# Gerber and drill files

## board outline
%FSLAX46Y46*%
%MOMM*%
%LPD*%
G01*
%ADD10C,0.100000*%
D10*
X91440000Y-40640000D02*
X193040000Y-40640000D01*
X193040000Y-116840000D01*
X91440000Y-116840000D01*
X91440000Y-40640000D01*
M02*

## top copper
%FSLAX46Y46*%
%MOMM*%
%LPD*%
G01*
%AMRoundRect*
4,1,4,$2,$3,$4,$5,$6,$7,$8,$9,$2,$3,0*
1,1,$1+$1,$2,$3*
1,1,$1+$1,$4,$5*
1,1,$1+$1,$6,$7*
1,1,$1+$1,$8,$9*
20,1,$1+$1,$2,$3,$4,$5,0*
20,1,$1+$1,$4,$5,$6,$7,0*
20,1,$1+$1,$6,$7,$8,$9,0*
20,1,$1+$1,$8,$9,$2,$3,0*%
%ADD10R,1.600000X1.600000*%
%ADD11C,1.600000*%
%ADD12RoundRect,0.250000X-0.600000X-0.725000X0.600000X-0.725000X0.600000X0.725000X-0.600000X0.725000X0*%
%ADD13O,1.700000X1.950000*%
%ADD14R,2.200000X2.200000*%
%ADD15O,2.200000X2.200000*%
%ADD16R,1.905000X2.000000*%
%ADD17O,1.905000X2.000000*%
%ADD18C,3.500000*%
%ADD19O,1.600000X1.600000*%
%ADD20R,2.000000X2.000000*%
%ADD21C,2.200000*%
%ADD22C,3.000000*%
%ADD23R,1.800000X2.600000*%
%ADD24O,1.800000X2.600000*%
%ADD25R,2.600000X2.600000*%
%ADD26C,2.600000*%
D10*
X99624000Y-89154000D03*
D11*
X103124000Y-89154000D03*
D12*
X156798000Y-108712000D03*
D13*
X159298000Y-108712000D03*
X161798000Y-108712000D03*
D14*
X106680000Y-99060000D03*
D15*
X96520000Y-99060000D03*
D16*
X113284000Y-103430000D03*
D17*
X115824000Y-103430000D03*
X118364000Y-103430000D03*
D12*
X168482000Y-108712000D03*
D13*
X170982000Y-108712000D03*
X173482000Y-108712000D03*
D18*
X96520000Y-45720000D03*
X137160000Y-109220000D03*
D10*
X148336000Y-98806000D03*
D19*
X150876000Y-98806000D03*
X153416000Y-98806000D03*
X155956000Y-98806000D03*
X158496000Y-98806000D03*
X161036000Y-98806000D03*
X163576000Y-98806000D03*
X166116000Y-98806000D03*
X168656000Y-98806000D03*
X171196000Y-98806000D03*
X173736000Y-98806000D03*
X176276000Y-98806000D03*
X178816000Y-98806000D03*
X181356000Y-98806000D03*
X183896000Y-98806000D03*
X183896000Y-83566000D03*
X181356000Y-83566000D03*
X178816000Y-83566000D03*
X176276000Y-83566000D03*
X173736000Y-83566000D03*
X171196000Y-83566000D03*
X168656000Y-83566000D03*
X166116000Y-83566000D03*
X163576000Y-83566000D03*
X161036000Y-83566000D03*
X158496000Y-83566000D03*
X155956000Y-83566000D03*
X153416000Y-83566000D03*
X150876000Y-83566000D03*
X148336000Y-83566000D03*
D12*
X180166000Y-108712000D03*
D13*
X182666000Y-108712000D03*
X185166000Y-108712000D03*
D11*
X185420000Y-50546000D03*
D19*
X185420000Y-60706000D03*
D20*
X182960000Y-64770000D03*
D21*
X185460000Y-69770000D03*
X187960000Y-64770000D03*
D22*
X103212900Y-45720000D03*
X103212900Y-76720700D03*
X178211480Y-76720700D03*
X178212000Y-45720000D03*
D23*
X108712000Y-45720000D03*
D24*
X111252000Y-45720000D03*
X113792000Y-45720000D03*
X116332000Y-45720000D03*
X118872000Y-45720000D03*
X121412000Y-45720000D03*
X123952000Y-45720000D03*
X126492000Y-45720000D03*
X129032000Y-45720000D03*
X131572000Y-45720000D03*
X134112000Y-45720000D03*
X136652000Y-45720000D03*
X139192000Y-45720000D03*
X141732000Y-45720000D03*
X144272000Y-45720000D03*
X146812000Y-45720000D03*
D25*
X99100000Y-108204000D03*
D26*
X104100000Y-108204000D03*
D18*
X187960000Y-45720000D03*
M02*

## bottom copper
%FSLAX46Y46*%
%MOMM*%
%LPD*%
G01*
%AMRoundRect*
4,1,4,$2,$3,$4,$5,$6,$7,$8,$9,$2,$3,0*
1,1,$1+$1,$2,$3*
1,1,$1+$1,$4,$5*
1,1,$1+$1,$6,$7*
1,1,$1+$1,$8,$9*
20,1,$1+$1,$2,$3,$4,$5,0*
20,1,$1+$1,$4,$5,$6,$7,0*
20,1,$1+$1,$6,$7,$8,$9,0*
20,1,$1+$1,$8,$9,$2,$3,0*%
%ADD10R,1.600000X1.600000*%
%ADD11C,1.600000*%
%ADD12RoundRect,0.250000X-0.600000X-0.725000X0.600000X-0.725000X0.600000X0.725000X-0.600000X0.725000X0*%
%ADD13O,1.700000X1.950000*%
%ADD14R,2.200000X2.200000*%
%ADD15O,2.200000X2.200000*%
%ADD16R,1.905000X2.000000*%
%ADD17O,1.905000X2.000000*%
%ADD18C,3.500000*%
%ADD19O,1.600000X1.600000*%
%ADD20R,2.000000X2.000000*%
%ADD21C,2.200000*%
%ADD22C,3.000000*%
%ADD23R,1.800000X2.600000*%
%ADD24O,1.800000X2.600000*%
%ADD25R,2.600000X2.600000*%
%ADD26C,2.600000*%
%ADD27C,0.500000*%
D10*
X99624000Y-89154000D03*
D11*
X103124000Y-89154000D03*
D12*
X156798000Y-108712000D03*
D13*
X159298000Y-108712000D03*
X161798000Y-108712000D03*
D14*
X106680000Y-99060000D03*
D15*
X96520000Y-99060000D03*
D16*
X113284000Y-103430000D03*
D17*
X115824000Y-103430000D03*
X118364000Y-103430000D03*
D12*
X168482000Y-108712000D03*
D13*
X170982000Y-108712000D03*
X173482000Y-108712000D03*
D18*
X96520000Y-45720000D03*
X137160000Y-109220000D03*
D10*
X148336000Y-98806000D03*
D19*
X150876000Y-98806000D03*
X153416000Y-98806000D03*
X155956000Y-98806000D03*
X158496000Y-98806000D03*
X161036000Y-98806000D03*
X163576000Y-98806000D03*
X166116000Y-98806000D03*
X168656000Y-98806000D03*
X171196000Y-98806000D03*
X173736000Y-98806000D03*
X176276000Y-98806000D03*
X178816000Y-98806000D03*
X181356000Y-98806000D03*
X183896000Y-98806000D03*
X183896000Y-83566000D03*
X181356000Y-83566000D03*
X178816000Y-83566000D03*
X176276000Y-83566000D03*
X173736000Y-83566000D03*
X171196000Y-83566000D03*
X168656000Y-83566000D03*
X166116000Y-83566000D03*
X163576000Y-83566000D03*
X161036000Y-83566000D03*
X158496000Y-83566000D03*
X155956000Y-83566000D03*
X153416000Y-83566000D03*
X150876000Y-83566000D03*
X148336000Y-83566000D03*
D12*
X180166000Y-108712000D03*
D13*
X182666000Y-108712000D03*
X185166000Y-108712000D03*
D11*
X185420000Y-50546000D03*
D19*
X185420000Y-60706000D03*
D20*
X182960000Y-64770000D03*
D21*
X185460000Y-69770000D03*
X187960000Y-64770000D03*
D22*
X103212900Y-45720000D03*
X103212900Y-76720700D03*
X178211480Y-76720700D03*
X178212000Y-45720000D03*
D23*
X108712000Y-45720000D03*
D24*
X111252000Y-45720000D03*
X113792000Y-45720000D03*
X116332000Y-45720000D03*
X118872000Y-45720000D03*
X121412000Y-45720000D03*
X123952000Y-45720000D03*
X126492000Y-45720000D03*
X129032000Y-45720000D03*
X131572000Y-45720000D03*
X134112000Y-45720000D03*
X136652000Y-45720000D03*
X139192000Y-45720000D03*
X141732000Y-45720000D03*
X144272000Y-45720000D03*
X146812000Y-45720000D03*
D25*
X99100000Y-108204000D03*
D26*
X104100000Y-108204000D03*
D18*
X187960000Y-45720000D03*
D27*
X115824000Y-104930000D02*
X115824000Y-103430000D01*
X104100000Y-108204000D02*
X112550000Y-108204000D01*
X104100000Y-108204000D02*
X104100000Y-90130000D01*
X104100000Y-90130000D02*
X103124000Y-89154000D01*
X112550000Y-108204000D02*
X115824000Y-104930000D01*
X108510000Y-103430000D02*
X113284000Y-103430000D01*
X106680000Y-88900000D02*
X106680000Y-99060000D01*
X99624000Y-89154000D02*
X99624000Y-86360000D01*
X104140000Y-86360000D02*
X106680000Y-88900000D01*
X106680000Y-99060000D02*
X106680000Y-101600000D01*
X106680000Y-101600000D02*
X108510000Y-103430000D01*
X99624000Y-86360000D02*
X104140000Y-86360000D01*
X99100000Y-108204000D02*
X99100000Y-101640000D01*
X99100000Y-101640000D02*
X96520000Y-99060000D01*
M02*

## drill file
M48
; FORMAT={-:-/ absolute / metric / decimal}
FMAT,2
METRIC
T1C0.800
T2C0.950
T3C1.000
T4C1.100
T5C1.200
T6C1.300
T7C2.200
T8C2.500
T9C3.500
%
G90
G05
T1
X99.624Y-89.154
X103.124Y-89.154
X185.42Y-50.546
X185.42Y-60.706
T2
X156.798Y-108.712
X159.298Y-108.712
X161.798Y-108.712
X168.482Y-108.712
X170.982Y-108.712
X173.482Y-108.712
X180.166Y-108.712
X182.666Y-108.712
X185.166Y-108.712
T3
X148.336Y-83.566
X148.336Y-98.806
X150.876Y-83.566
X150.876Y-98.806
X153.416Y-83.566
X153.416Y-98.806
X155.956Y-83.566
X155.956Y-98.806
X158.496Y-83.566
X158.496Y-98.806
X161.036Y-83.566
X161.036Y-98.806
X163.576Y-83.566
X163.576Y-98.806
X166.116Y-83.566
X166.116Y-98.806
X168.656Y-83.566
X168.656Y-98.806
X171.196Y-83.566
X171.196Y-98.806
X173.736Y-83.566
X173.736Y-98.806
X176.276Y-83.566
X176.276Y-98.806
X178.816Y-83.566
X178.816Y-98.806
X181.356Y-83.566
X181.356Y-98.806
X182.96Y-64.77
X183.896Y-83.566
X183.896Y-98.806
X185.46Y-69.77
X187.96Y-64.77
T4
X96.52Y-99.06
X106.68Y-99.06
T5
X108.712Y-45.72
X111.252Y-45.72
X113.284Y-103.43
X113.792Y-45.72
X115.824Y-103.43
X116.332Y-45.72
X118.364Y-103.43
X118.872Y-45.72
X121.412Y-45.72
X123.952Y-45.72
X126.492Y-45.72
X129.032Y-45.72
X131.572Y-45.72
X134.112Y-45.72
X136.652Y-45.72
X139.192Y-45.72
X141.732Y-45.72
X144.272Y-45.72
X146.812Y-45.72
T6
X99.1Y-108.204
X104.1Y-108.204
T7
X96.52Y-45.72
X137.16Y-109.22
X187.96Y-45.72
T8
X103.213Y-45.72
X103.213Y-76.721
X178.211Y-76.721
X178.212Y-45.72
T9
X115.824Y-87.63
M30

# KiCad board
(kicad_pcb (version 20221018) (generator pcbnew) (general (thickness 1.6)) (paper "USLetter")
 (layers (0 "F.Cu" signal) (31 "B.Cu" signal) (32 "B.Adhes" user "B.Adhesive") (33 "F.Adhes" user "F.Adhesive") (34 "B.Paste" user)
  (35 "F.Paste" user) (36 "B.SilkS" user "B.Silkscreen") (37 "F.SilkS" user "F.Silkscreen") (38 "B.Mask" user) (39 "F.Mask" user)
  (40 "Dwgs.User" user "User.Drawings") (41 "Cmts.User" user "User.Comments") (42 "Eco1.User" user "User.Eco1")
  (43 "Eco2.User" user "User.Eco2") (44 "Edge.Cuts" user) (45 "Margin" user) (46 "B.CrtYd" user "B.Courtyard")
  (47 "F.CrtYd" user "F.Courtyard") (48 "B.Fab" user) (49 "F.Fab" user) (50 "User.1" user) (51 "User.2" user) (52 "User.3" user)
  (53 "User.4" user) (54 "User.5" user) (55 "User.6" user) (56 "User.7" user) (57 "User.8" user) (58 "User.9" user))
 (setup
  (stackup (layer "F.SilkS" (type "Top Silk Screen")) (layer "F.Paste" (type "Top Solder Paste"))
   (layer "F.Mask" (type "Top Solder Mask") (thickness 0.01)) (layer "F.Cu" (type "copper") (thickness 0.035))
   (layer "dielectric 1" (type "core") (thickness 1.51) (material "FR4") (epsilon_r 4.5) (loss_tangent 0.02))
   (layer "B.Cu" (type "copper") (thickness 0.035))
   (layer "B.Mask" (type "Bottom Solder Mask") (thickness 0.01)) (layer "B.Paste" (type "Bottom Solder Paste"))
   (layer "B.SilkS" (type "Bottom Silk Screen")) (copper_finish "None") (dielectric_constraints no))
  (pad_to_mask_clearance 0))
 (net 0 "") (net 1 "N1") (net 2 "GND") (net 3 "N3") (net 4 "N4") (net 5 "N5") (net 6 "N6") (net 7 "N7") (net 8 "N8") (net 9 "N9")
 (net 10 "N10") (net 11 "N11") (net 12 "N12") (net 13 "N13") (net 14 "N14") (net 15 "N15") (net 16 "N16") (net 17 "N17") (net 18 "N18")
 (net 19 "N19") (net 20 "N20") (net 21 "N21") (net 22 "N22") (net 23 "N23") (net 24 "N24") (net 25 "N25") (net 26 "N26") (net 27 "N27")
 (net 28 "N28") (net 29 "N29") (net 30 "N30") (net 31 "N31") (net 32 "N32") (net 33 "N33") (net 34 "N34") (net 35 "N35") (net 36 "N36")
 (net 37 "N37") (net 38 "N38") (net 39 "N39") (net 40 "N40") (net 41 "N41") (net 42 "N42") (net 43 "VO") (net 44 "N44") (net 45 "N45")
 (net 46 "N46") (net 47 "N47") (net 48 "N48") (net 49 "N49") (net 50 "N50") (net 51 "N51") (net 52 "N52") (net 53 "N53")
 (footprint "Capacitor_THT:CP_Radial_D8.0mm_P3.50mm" (layer "F.Cu") (at 99.624 89.154)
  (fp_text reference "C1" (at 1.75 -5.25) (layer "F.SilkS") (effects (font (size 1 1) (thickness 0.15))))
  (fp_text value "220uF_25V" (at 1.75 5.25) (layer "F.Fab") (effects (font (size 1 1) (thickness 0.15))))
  (pad "1" thru_hole rect (at 0 0) (size 1.6 1.6) (drill 0.8) (layers "*.Cu" "*.Mask") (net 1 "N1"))
  (pad "2" thru_hole circle (at 3.5 0) (size 1.6 1.6) (drill 0.8) (layers "*.Cu" "*.Mask") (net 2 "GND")))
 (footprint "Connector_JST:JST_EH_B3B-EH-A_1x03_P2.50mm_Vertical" (layer "F.Cu") (at 156.798 108.712)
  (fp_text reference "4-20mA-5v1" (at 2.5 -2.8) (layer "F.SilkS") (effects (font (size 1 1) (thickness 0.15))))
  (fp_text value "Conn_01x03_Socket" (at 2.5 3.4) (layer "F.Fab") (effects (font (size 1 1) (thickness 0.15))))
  (pad "1" thru_hole roundrect (at 0 0) (size 1.7 1.95) (drill 0.95) (layers "*.Cu" "*.Mask") (roundrect_rratio 0.147059) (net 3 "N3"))
  (pad "2" thru_hole oval (at 2.5 0) (size 1.7 1.95) (drill 0.95) (layers "*.Cu" "*.Mask") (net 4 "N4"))
  (pad "3" thru_hole oval (at 5 0) (size 1.7 1.95) (drill 0.95) (layers "*.Cu" "*.Mask") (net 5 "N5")))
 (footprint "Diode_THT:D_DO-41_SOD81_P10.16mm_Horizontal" (layer "F.Cu") (at 106.68 99.06 180)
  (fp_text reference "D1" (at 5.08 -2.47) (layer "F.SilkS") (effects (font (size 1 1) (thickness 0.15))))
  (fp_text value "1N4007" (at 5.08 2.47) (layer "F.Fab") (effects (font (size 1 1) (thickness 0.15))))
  (pad "1" thru_hole rect (at 0 0 180) (size 2.2 2.2) (drill 1.1) (layers "*.Cu" "*.Mask") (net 1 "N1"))
  (pad "2" thru_hole oval (at 10.16 0 180) (size 2.2 2.2) (drill 1.1) (layers "*.Cu" "*.Mask") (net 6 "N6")))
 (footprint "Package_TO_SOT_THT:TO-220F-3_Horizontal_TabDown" (layer "F.Cu") (at 113.284 103.43)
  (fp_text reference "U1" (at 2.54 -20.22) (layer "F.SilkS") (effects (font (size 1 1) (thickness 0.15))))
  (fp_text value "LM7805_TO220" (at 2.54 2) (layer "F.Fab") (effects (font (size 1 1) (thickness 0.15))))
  (pad "" np_thru_hole oval (at 2.54 -15.8) (size 3.5 3.5) (drill 3.5) (layers "*.Cu" "*.Mask"))
  (pad "1" thru_hole rect (at 0 0) (size 1.905 2) (drill 1.2) (layers "*.Cu" "*.Mask") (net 1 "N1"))
  (pad "2" thru_hole oval (at 2.54 0) (size 1.905 2) (drill 1.2) (layers "*.Cu" "*.Mask") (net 2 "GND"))
  (pad "3" thru_hole oval (at 5.08 0) (size 1.905 2) (drill 1.2) (layers "*.Cu" "*.Mask") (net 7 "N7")))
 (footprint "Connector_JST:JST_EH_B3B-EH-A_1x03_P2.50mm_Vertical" (layer "F.Cu") (at 168.482 108.712)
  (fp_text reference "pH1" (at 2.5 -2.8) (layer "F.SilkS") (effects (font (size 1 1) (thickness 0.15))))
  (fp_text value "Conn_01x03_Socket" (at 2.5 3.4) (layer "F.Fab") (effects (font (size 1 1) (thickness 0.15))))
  (pad "1" thru_hole roundrect (at 0 0) (size 1.7 1.95) (drill 0.95) (layers "*.Cu" "*.Mask") (roundrect_rratio 0.147059) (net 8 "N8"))
  (pad "2" thru_hole oval (at 2.5 0) (size 1.7 1.95) (drill 0.95) (layers "*.Cu" "*.Mask") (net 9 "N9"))
  (pad "3" thru_hole oval (at 5 0) (size 1.7 1.95) (drill 0.95) (layers "*.Cu" "*.Mask") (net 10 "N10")))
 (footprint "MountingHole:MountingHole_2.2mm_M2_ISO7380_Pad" (layer "F.Cu") (at 96.52 45.72)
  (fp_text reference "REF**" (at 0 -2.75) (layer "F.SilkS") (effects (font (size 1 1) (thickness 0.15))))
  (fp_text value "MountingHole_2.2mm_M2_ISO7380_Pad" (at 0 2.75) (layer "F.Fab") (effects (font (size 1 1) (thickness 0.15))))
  (pad "1" thru_hole circle (at 0 0) (size 3.5 3.5) (drill 2.2) (layers "*.Cu" "*.Mask")))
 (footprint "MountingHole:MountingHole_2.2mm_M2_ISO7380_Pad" (layer "F.Cu") (at 137.16 109.22)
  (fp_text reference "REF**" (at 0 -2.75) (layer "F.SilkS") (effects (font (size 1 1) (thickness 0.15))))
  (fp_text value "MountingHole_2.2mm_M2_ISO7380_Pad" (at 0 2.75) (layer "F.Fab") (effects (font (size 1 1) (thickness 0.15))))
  (pad "1" thru_hole circle (at 0 0) (size 3.5 3.5) (drill 2.2) (layers "*.Cu" "*.Mask")))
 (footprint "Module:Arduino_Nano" (layer "F.Cu") (at 148.336 98.806 90)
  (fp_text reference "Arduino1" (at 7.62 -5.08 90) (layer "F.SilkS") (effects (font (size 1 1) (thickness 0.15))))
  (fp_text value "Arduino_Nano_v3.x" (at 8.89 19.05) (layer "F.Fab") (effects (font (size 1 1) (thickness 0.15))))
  (pad "1" thru_hole rect (at 0 0 90) (size 1.6 1.6) (drill 1) (layers "*.Cu" "*.Mask") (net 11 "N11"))
  (pad "2" thru_hole oval (at 0 2.54 90) (size 1.6 1.6) (drill 1) (layers "*.Cu" "*.Mask") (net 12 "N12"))
  (pad "3" thru_hole oval (at 0 5.08 90) (size 1.6 1.6) (drill 1) (layers "*.Cu" "*.Mask") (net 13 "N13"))
  (pad "4" thru_hole oval (at 0 7.62 90) (size 1.6 1.6) (drill 1) (layers "*.Cu" "*.Mask") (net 2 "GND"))
  (pad "5" thru_hole oval (at 0 10.16 90) (size 1.6 1.6) (drill 1) (layers "*.Cu" "*.Mask") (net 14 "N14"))
  (pad "6" thru_hole oval (at 0 12.7 90) (size 1.6 1.6) (drill 1) (layers "*.Cu" "*.Mask") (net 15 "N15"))
  (pad "7" thru_hole oval (at 0 15.24 90) (size 1.6 1.6) (drill 1) (layers "*.Cu" "*.Mask") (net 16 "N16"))
  (pad "8" thru_hole oval (at 0 17.78 90) (size 1.6 1.6) (drill 1) (layers "*.Cu" "*.Mask") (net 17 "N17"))
  (pad "9" thru_hole oval (at 0 20.32 90) (size 1.6 1.6) (drill 1) (layers "*.Cu" "*.Mask") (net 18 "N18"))
  (pad "10" thru_hole oval (at 0 22.86 90) (size 1.6 1.6) (drill 1) (layers "*.Cu" "*.Mask") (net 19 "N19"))
  (pad "11" thru_hole oval (at 0 25.4 90) (size 1.6 1.6) (drill 1) (layers "*.Cu" "*.Mask") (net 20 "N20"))
  (pad "12" thru_hole oval (at 0 27.94 90) (size 1.6 1.6) (drill 1) (layers "*.Cu" "*.Mask") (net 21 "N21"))
  (pad "13" thru_hole oval (at 0 30.48 90) (size 1.6 1.6) (drill 1) (layers "*.Cu" "*.Mask") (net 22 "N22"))
  (pad "14" thru_hole oval (at 0 33.02 90) (size 1.6 1.6) (drill 1) (layers "*.Cu" "*.Mask") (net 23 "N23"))
  (pad "15" thru_hole oval (at 0 35.56 90) (size 1.6 1.6) (drill 1) (layers "*.Cu" "*.Mask") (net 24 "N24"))
  (pad "16" thru_hole oval (at 15.24 35.56 90) (size 1.6 1.6) (drill 1) (layers "*.Cu" "*.Mask") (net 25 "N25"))
  (pad "17" thru_hole oval (at 15.24 33.02 90) (size 1.6 1.6) (drill 1) (layers "*.Cu" "*.Mask") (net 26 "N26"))
  (pad "18" thru_hole oval (at 15.24 30.48 90) (size 1.6 1.6) (drill 1) (layers "*.Cu" "*.Mask") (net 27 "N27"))
  (pad "19" thru_hole oval (at 15.24 27.94 90) (size 1.6 1.6) (drill 1) (layers "*.Cu" "*.Mask") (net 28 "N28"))
  (pad "20" thru_hole oval (at 15.24 25.4 90) (size 1.6 1.6) (drill 1) (layers "*.Cu" "*.Mask") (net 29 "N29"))
  (pad "21" thru_hole oval (at 15.24 22.86 90) (size 1.6 1.6) (drill 1) (layers "*.Cu" "*.Mask") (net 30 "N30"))
  (pad "22" thru_hole oval (at 15.24 20.32 90) (size 1.6 1.6) (drill 1) (layers "*.Cu" "*.Mask") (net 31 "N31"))
  (pad "23" thru_hole oval (at 15.24 17.78 90) (size 1.6 1.6) (drill 1) (layers "*.Cu" "*.Mask") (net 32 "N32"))
  (pad "24" thru_hole oval (at 15.24 15.24 90) (size 1.6 1.6) (drill 1) (layers "*.Cu" "*.Mask") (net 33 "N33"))
  (pad "25" thru_hole oval (at 15.24 12.7 90) (size 1.6 1.6) (drill 1) (layers "*.Cu" "*.Mask") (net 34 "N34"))
  (pad "26" thru_hole oval (at 15.24 10.16 90) (size 1.6 1.6) (drill 1) (layers "*.Cu" "*.Mask") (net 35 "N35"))
  (pad "27" thru_hole oval (at 15.24 7.62 90) (size 1.6 1.6) (drill 1) (layers "*.Cu" "*.Mask") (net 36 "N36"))
  (pad "28" thru_hole oval (at 15.24 5.08 90) (size 1.6 1.6) (drill 1) (layers "*.Cu" "*.Mask") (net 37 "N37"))
  (pad "29" thru_hole oval (at 15.24 2.54 90) (size 1.6 1.6) (drill 1) (layers "*.Cu" "*.Mask") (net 2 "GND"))
  (pad "30" thru_hole oval (at 15.24 0 90) (size 1.6 1.6) (drill 1) (layers "*.Cu" "*.Mask") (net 7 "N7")))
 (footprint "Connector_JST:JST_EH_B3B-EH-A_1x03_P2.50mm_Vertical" (layer "F.Cu") (at 180.166 108.712)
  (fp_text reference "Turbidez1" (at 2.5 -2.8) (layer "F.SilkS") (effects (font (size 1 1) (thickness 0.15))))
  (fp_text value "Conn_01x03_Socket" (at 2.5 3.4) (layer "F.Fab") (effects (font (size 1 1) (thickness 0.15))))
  (pad "1" thru_hole roundrect (at 0 0) (size 1.7 1.95) (drill 0.95) (layers "*.Cu" "*.Mask") (roundrect_rratio 0.147059) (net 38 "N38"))
  (pad "2" thru_hole oval (at 2.5 0) (size 1.7 1.95) (drill 0.95) (layers "*.Cu" "*.Mask") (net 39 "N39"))
  (pad "3" thru_hole oval (at 5 0) (size 1.7 1.95) (drill 0.95) (layers "*.Cu" "*.Mask") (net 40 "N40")))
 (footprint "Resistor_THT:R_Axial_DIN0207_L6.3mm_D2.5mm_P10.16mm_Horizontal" (layer "F.Cu") (at 185.42 50.546 -90)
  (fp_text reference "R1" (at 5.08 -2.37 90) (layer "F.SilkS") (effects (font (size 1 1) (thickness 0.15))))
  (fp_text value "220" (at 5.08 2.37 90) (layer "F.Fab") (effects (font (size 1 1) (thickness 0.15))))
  (pad "1" thru_hole circle (at 0 0 270) (size 1.6 1.6) (drill 0.8) (layers "*.Cu" "*.Mask") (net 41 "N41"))
  (pad "2" thru_hole oval (at 10.16 0 270) (size 1.6 1.6) (drill 0.8) (layers "*.Cu" "*.Mask") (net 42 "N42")))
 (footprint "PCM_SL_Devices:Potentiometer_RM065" (layer "F.Cu") (at 185.49 66.8)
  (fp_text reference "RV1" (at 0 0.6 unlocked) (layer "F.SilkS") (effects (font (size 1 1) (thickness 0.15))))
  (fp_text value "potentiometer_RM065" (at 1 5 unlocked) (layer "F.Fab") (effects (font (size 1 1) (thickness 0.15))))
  (pad "1" thru_hole rect (at -2.53 -2.03) (size 2 2) (drill 1) (layers "*.Cu" "*.Mask") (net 36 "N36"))
  (pad "2" thru_hole circle (at -0.03 2.97) (size 2.2 2.2) (drill 1) (layers "*.Cu" "*.Mask") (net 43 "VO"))
  (pad "3" thru_hole circle (at 2.47 -2.03) (size 2.2 2.2) (drill 1) (layers "*.Cu" "*.Mask") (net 2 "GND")))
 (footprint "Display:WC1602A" (layer "F.Cu") (at 108.712 45.72)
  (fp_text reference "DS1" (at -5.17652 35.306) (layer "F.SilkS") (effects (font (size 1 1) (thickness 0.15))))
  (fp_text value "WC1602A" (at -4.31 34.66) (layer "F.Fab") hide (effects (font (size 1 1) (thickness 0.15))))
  (pad "" thru_hole circle (at -5.4991 0) (size 3 3) (drill 2.5) (layers "*.Cu" "*.Mask"))
  (pad "" thru_hole circle (at -5.4991 31.0007) (size 3 3) (drill 2.5) (layers "*.Cu" "*.Mask"))
  (pad "" thru_hole circle (at 69.49948 31.0007) (size 3 3) (drill 2.5) (layers "*.Cu" "*.Mask"))
  (pad "" thru_hole circle (at 69.5 0) (size 3 3) (drill 2.5) (layers "*.Cu" "*.Mask"))
  (pad "1" thru_hole rect (at 0 0) (size 1.8 2.6) (drill 1.2) (layers "*.Cu" "*.Mask") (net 2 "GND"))
  (pad "2" thru_hole oval (at 2.54 0) (size 1.8 2.6) (drill 1.2) (layers "*.Cu" "*.Mask") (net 36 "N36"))
  (pad "3" thru_hole oval (at 5.08 0) (size 1.8 2.6) (drill 1.2) (layers "*.Cu" "*.Mask") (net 43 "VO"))
  (pad "4" thru_hole oval (at 7.62 0) (size 1.8 2.6) (drill 1.2) (layers "*.Cu" "*.Mask") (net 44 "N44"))
  (pad "5" thru_hole oval (at 10.16 0) (size 1.8 2.6) (drill 1.2) (layers "*.Cu" "*.Mask") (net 15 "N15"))
  (pad "6" thru_hole oval (at 12.7 0) (size 1.8 2.6) (drill 1.2) (layers "*.Cu" "*.Mask") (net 14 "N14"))
  (pad "7" thru_hole oval (at 15.24 0) (size 1.8 2.6) (drill 1.2) (layers "*.Cu" "*.Mask") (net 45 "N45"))
  (pad "8" thru_hole oval (at 17.78 0) (size 1.8 2.6) (drill 1.2) (layers "*.Cu" "*.Mask") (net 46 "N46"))
  (pad "9" thru_hole oval (at 20.32 0) (size 1.8 2.6) (drill 1.2) (layers "*.Cu" "*.Mask") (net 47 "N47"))
  (pad "10" thru_hole oval (at 22.86 0) (size 1.8 2.6) (drill 1.2) (layers "*.Cu" "*.Mask") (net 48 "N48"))
  (pad "11" thru_hole oval (at 25.4 0) (size 1.8 2.6) (drill 1.2) (layers "*.Cu" "*.Mask") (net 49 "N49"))
  (pad "12" thru_hole oval (at 27.94 0) (size 1.8 2.6) (drill 1.2) (layers "*.Cu" "*.Mask") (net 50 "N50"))
  (pad "13" thru_hole oval (at 30.48 0) (size 1.8 2.6) (drill 1.2) (layers "*.Cu" "*.Mask") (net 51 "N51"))
  (pad "14" thru_hole oval (at 33.02 0) (size 1.8 2.6) (drill 1.2) (layers "*.Cu" "*.Mask") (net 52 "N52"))
  (pad "15" thru_hole oval (at 35.56 0) (size 1.8 2.6) (drill 1.2) (layers "*.Cu" "*.Mask") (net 41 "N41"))
  (pad "16" thru_hole oval (at 38.1 0) (size 1.8 2.6) (drill 1.2) (layers "*.Cu" "*.Mask") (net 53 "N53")))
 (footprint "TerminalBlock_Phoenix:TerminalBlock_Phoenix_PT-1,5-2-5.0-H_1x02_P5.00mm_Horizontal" (layer "F.Cu") (at 99.1 108.204)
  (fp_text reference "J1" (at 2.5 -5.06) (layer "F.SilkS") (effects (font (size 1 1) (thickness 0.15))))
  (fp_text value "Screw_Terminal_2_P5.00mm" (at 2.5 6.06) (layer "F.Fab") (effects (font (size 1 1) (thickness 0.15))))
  (pad "1" thru_hole rect (at 0 0) (size 2.6 2.6) (drill 1.3) (layers "*.Cu" "*.Mask") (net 6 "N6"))
  (pad "2" thru_hole circle (at 5 0) (size 2.6 2.6) (drill 1.3) (layers "*.Cu" "*.Mask") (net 2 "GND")))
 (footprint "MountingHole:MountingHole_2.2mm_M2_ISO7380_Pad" (layer "F.Cu") (at 187.96 45.72)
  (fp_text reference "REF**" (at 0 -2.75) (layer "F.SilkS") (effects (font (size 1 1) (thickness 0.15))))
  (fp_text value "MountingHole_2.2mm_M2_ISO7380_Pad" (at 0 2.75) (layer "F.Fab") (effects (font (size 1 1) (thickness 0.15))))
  (pad "1" thru_hole circle (at 0 0) (size 3.5 3.5) (drill 2.2) (layers "*.Cu" "*.Mask")))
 (gr_rect (start 105.31 137.08) (end 105.31 137.08) (stroke (width 0.1) (type default)) (fill none) (layer "Edge.Cuts"))
 (gr_rect (start 91.44 40.64) (end 193.04 116.84) (stroke (width 0.1) (type default)) (fill none) (layer "Edge.Cuts"))
 (segment (start 115.824 104.93) (end 115.824 103.43) (width 0.5) (layer "B.Cu") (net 2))
 (segment (start 104.1 108.204) (end 112.55 108.204) (width 0.5) (layer "B.Cu") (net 2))
 (segment (start 104.1 108.204) (end 104.1 90.13) (width 0.5) (layer "B.Cu") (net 2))
 (segment (start 104.1 90.13) (end 103.124 89.154) (width 0.5) (layer "B.Cu") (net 2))
 (segment (start 112.55 108.204) (end 115.824 104.93) (width 0.5) (layer "B.Cu") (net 2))
 (segment (start 108.51 103.43) (end 113.284 103.43) (width 0.5) (layer "B.Cu") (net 1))
 (segment (start 106.68 88.9) (end 106.68 99.06) (width 0.5) (layer "B.Cu") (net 1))
 (segment (start 99.624 89.154) (end 99.624 86.36) (width 0.5) (layer "B.Cu") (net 1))
 (segment (start 104.14 86.36) (end 106.68 88.9) (width 0.5) (layer "B.Cu") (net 1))
 (segment (start 106.68 99.06) (end 106.68 101.6) (width 0.5) (layer "B.Cu") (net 1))
 (segment (start 106.68 101.6) (end 108.51 103.43) (width 0.5) (layer "B.Cu") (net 1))
 (segment (start 99.624 86.36) (end 104.14 86.36) (width 0.5) (layer "B.Cu") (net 1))
 (segment (start 99.1 108.204) (end 99.1 101.64) (width 0.5) (layer "B.Cu") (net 6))
 (segment (start 99.1 101.64) (end 96.52 99.06) (width 0.5) (layer "B.Cu") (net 6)))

